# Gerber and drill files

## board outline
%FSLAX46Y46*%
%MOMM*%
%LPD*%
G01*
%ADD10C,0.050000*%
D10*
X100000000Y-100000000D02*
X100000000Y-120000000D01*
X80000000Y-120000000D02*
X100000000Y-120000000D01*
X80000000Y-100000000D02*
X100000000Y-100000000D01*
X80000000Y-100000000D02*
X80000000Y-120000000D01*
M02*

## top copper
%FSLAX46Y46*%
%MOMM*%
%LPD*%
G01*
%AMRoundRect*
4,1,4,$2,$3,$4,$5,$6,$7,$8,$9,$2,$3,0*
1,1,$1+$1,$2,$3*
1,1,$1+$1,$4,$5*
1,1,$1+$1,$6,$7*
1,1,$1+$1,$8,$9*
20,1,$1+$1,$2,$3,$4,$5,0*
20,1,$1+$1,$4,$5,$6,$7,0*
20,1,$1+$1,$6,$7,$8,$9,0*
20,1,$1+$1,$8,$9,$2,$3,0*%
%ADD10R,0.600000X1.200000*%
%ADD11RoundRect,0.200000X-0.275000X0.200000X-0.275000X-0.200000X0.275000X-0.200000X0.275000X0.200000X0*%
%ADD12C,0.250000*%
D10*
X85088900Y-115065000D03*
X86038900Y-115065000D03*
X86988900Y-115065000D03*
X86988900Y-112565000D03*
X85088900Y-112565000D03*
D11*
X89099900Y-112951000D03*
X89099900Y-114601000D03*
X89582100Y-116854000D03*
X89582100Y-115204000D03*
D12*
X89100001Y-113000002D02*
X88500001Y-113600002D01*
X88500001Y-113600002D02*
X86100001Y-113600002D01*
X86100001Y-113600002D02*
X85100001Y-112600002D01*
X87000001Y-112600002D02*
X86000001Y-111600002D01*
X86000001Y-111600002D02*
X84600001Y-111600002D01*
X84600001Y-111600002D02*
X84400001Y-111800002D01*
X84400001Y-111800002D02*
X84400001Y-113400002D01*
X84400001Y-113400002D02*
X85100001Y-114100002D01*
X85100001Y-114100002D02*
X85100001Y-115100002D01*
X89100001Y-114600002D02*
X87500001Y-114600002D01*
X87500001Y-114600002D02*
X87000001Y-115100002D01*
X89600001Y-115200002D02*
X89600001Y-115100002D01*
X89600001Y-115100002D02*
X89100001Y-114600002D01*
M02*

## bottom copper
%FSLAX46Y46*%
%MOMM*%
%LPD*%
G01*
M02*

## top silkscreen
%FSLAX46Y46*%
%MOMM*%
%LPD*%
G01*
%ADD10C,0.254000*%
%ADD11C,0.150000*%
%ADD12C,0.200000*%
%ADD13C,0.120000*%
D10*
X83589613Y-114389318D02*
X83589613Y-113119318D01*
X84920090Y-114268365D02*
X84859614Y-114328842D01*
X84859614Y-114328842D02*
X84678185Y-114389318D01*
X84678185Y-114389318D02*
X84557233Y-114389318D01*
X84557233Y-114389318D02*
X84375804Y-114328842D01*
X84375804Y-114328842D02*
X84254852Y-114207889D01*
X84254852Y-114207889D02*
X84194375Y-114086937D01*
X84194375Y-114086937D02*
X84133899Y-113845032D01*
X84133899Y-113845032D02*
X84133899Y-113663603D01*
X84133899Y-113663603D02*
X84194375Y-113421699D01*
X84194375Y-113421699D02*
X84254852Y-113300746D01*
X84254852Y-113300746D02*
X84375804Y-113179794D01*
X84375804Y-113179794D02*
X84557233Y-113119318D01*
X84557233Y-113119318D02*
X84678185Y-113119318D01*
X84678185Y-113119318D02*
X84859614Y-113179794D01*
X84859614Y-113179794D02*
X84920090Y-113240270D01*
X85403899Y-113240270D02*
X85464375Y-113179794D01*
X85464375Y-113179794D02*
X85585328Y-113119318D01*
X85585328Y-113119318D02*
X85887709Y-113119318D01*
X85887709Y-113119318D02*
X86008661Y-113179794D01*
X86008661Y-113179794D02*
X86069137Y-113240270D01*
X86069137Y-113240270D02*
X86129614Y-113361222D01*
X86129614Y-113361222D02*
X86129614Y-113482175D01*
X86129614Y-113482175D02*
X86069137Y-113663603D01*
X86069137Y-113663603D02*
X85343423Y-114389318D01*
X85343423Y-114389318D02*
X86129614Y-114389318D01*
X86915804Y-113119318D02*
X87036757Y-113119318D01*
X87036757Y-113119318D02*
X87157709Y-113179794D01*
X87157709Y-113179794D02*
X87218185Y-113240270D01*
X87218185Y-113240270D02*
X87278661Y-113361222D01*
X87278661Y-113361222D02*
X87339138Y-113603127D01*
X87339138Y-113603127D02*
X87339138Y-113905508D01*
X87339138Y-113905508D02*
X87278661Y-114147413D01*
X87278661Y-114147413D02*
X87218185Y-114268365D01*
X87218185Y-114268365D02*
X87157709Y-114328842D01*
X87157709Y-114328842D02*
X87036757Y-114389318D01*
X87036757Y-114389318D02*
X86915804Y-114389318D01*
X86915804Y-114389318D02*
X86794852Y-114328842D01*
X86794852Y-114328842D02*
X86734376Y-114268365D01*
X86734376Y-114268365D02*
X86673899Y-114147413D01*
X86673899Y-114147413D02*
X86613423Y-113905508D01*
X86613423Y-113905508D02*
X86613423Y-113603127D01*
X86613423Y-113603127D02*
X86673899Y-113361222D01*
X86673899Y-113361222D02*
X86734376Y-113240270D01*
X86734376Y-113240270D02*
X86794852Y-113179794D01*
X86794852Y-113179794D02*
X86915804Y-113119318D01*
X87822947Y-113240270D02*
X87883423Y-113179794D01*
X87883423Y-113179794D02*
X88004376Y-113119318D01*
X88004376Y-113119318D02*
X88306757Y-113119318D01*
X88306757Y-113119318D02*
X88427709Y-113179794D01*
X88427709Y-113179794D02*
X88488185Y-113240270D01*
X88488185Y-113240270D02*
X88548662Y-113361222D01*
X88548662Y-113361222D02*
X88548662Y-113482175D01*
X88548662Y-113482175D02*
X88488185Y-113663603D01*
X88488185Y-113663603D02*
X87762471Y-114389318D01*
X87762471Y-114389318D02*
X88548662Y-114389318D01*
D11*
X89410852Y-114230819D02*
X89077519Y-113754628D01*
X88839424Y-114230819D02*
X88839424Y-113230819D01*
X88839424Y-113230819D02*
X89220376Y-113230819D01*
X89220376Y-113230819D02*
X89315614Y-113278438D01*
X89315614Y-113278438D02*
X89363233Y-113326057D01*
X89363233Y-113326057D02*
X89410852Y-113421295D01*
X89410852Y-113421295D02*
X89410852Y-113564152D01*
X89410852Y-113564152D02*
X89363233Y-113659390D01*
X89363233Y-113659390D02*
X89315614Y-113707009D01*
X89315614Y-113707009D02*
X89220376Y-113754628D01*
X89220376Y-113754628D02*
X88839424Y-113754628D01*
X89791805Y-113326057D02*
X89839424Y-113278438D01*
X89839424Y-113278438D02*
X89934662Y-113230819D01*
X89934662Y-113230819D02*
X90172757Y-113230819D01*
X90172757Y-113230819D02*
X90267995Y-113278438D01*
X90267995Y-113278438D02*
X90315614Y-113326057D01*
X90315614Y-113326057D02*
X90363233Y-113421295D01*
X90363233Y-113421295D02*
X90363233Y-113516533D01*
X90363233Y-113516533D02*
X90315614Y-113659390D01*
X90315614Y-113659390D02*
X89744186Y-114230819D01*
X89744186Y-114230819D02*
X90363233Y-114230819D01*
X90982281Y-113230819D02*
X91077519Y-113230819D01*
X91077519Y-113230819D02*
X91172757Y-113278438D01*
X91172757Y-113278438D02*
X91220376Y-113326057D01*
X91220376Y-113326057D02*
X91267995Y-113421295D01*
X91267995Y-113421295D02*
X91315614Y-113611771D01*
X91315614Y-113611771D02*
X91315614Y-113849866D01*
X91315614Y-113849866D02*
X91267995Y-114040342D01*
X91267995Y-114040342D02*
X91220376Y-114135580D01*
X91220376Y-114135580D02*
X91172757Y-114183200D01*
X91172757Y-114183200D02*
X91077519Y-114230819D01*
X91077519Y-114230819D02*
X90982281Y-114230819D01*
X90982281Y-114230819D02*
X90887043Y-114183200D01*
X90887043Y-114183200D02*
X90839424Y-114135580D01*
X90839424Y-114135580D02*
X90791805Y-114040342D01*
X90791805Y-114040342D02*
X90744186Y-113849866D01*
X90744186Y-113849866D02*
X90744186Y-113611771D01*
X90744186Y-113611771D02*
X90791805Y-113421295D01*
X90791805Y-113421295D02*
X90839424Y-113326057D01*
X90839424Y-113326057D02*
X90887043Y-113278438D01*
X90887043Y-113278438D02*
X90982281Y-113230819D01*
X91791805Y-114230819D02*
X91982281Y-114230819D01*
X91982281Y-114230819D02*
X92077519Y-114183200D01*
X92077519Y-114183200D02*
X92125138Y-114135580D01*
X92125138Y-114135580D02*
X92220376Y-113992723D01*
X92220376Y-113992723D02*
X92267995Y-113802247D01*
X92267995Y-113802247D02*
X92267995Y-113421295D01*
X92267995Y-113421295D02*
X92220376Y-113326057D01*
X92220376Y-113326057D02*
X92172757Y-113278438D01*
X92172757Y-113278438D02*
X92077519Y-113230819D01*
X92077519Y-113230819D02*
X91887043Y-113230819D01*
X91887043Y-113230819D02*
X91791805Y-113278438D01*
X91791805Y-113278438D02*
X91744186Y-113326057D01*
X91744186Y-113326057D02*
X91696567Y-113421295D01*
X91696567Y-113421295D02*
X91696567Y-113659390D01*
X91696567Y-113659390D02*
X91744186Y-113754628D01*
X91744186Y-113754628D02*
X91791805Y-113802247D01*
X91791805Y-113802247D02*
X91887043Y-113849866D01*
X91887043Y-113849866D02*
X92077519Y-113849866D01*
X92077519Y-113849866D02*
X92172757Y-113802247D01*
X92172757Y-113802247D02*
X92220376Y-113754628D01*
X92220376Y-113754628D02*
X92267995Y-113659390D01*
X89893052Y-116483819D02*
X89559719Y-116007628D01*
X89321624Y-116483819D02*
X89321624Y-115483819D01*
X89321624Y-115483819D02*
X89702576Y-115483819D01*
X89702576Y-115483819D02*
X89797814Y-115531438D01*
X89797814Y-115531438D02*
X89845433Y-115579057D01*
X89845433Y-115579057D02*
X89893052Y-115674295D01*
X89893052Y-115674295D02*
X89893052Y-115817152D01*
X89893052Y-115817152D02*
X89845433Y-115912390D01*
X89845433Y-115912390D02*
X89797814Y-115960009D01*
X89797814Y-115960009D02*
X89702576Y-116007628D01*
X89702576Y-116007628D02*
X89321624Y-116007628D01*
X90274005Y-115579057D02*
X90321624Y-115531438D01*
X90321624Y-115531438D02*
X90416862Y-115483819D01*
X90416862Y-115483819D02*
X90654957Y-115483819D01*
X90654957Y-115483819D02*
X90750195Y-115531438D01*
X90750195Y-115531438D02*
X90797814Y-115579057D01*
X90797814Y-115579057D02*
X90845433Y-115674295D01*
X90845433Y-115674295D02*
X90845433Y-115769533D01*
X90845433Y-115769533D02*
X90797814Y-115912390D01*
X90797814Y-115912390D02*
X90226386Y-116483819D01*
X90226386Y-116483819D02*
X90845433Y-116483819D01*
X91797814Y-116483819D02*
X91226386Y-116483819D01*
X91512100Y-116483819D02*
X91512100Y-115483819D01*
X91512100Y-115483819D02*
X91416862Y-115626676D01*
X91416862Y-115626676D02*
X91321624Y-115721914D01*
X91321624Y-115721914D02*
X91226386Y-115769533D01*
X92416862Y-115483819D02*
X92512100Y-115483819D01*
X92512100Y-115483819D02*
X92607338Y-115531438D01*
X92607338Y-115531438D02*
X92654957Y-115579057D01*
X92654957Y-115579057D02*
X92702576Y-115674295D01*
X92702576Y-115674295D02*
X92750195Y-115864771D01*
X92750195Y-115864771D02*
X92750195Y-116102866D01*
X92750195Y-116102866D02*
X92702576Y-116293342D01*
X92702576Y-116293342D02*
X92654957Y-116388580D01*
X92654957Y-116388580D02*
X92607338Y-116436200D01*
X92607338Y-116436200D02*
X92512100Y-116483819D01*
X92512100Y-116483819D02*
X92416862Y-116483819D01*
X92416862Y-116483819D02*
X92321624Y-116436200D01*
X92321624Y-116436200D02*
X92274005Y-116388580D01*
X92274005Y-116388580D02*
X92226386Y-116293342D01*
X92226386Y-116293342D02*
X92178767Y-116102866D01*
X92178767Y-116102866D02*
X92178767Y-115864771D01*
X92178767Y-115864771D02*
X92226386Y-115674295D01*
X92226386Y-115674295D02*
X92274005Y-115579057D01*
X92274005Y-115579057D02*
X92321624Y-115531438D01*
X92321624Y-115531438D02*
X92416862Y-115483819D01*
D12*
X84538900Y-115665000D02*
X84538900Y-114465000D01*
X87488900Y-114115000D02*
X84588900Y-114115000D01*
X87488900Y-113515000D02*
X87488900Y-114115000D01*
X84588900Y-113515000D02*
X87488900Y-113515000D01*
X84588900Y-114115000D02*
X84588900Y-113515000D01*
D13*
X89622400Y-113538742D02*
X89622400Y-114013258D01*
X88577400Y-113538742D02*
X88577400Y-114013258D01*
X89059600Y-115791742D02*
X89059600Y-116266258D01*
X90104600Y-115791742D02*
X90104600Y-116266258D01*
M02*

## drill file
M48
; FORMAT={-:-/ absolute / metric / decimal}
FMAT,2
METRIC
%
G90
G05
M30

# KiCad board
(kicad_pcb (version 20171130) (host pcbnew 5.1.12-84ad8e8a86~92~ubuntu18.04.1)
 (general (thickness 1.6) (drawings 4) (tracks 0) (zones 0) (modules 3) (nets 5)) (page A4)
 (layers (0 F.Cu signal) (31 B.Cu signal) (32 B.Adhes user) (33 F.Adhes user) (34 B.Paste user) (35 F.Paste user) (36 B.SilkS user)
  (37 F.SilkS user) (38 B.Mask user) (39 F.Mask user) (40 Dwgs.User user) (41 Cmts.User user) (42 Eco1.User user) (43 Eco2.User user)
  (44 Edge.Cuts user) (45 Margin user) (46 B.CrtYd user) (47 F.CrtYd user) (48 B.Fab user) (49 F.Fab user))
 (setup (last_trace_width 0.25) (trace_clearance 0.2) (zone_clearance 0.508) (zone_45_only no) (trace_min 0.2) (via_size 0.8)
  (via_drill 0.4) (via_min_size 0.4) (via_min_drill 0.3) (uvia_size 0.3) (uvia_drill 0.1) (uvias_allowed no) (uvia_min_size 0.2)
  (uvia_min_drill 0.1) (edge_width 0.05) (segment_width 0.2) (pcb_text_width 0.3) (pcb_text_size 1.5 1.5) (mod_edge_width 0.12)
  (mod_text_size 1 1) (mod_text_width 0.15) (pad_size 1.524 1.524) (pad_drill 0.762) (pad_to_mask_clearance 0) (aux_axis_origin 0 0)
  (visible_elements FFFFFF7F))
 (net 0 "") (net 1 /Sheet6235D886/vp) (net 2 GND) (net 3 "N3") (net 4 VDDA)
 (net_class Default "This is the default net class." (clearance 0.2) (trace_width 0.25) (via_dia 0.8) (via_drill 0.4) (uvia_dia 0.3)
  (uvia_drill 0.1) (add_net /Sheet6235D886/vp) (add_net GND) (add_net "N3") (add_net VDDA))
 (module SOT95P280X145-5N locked (layer F.Cu) (at 86.038900 113.815000 90.000000)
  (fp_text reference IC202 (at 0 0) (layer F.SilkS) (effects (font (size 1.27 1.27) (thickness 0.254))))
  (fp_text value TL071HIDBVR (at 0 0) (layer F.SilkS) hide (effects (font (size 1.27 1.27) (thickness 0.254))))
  (fp_line (start -1.85 -1.5) (end -0.65 -1.5) (layer F.SilkS) (width 0.2))
  (fp_line (start -0.3 1.45) (end -0.3 -1.45) (layer F.SilkS) (width 0.2))
  (fp_line (start 0.3 1.45) (end -0.3 1.45) (layer F.SilkS) (width 0.2))
  (fp_line (start 0.3 -1.45) (end 0.3 1.45) (layer F.SilkS) (width 0.2))
  (fp_line (start -0.3 -1.45) (end 0.3 -1.45) (layer F.SilkS) (width 0.2))
  (pad 1 smd rect (at -1.25 -0.95 180.000000) (size 0.6 1.2) (layers F.Cu F.Mask F.Paste) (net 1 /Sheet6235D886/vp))
  (pad 2 smd rect (at -1.25 0 180.000000) (size 0.6 1.2) (layers F.Cu F.Mask F.Paste) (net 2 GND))
  (pad 3 smd rect (at -1.25 0.95 180.000000) (size 0.6 1.2) (layers F.Cu F.Mask F.Paste) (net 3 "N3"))
  (pad 4 smd rect (at 1.25 0.95 180.000000) (size 0.6 1.2) (layers F.Cu F.Mask F.Paste) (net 1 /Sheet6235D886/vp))
  (pad 5 smd rect (at 1.25 -0.95 180.000000) (size 0.6 1.2) (layers F.Cu F.Mask F.Paste) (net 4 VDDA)))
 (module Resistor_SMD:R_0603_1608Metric (layer F.Cu) (at 89.099900 113.776000 270.000000)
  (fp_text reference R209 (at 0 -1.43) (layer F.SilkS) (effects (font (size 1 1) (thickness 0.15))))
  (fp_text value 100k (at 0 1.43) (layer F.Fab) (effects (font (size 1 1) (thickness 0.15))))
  (fp_line (start -0.237258 -0.5225) (end 0.237258 -0.5225) (layer F.SilkS) (width 0.12))
  (fp_line (start -0.237258 0.5225) (end 0.237258 0.5225) (layer F.SilkS) (width 0.12))
  (pad 1 smd roundrect (at -0.825 0 270.000000) (size 0.8 0.95) (layers F.Cu F.Mask F.Paste) (roundrect_rratio 0.25) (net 4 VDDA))
  (pad 2 smd roundrect (at 0.825 0 270.000000) (size 0.8 0.95) (layers F.Cu F.Mask F.Paste) (roundrect_rratio 0.25) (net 3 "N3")))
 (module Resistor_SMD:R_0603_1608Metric (layer F.Cu) (at 89.582100 116.029000 270.000000)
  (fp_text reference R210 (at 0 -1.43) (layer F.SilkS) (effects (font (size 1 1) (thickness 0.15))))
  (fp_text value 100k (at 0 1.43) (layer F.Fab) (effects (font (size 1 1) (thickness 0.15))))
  (fp_line (start -0.237258 0.5225) (end 0.237258 0.5225) (layer F.SilkS) (width 0.12))
  (fp_line (start -0.237258 -0.5225) (end 0.237258 -0.5225) (layer F.SilkS) (width 0.12))
  (pad 2 smd roundrect (at 0.825 0 270.000000) (size 0.8 0.95) (layers F.Cu F.Mask F.Paste) (roundrect_rratio 0.25) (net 2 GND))
  (pad 1 smd roundrect (at -0.825 0 270.000000) (size 0.8 0.95) (layers F.Cu F.Mask F.Paste) (roundrect_rratio 0.25) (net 3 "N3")))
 (gr_line (start 100 100) (end 100 120) (layer Edge.Cuts) (width 0.05))
 (gr_line (start 80 120) (end 100 120) (layer Edge.Cuts) (width 0.05))
 (gr_line (start 80 100) (end 100 100) (layer Edge.Cuts) (width 0.05))
 (gr_line (start 80 100) (end 80 120) (layer Edge.Cuts) (width 0.05))
 (segment (start 89.100001 113.000002) (end 88.500001 113.600002) (width 0.250000) (layer F.Cu) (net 4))
 (segment (start 88.500001 113.600002) (end 86.100001 113.600002) (width 0.250000) (layer F.Cu) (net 4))
 (segment (start 86.100001 113.600002) (end 85.100001 112.600002) (width 0.250000) (layer F.Cu) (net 4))
 (segment (start 87.000001 112.600002) (end 86.000001 111.600002) (width 0.250000) (layer F.Cu) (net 1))
 (segment (start 86.000001 111.600002) (end 84.600001 111.600002) (width 0.250000) (layer F.Cu) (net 1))
 (segment (start 84.600001 111.600002) (end 84.400001 111.800002) (width 0.250000) (layer F.Cu) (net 1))
 (segment (start 84.400001 111.800002) (end 84.400001 113.400002) (width 0.250000) (layer F.Cu) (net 1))
 (segment (start 84.400001 113.400002) (end 85.100001 114.100002) (width 0.250000) (layer F.Cu) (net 1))
 (segment (start 85.100001 114.100002) (end 85.100001 115.100002) (width 0.250000) (layer F.Cu) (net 1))
 (segment (start 89.100001 114.600002) (end 87.500001 114.600002) (width 0.250000) (layer F.Cu) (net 3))
 (segment (start 87.500001 114.600002) (end 87.000001 115.100002) (width 0.250000) (layer F.Cu) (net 3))
 (segment (start 89.600001 115.200002) (end 89.600001 115.100002) (width 0.250000) (layer F.Cu) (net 3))
 (segment (start 89.600001 115.100002) (end 89.100001 114.600002) (width 0.250000) (layer F.Cu) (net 3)))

